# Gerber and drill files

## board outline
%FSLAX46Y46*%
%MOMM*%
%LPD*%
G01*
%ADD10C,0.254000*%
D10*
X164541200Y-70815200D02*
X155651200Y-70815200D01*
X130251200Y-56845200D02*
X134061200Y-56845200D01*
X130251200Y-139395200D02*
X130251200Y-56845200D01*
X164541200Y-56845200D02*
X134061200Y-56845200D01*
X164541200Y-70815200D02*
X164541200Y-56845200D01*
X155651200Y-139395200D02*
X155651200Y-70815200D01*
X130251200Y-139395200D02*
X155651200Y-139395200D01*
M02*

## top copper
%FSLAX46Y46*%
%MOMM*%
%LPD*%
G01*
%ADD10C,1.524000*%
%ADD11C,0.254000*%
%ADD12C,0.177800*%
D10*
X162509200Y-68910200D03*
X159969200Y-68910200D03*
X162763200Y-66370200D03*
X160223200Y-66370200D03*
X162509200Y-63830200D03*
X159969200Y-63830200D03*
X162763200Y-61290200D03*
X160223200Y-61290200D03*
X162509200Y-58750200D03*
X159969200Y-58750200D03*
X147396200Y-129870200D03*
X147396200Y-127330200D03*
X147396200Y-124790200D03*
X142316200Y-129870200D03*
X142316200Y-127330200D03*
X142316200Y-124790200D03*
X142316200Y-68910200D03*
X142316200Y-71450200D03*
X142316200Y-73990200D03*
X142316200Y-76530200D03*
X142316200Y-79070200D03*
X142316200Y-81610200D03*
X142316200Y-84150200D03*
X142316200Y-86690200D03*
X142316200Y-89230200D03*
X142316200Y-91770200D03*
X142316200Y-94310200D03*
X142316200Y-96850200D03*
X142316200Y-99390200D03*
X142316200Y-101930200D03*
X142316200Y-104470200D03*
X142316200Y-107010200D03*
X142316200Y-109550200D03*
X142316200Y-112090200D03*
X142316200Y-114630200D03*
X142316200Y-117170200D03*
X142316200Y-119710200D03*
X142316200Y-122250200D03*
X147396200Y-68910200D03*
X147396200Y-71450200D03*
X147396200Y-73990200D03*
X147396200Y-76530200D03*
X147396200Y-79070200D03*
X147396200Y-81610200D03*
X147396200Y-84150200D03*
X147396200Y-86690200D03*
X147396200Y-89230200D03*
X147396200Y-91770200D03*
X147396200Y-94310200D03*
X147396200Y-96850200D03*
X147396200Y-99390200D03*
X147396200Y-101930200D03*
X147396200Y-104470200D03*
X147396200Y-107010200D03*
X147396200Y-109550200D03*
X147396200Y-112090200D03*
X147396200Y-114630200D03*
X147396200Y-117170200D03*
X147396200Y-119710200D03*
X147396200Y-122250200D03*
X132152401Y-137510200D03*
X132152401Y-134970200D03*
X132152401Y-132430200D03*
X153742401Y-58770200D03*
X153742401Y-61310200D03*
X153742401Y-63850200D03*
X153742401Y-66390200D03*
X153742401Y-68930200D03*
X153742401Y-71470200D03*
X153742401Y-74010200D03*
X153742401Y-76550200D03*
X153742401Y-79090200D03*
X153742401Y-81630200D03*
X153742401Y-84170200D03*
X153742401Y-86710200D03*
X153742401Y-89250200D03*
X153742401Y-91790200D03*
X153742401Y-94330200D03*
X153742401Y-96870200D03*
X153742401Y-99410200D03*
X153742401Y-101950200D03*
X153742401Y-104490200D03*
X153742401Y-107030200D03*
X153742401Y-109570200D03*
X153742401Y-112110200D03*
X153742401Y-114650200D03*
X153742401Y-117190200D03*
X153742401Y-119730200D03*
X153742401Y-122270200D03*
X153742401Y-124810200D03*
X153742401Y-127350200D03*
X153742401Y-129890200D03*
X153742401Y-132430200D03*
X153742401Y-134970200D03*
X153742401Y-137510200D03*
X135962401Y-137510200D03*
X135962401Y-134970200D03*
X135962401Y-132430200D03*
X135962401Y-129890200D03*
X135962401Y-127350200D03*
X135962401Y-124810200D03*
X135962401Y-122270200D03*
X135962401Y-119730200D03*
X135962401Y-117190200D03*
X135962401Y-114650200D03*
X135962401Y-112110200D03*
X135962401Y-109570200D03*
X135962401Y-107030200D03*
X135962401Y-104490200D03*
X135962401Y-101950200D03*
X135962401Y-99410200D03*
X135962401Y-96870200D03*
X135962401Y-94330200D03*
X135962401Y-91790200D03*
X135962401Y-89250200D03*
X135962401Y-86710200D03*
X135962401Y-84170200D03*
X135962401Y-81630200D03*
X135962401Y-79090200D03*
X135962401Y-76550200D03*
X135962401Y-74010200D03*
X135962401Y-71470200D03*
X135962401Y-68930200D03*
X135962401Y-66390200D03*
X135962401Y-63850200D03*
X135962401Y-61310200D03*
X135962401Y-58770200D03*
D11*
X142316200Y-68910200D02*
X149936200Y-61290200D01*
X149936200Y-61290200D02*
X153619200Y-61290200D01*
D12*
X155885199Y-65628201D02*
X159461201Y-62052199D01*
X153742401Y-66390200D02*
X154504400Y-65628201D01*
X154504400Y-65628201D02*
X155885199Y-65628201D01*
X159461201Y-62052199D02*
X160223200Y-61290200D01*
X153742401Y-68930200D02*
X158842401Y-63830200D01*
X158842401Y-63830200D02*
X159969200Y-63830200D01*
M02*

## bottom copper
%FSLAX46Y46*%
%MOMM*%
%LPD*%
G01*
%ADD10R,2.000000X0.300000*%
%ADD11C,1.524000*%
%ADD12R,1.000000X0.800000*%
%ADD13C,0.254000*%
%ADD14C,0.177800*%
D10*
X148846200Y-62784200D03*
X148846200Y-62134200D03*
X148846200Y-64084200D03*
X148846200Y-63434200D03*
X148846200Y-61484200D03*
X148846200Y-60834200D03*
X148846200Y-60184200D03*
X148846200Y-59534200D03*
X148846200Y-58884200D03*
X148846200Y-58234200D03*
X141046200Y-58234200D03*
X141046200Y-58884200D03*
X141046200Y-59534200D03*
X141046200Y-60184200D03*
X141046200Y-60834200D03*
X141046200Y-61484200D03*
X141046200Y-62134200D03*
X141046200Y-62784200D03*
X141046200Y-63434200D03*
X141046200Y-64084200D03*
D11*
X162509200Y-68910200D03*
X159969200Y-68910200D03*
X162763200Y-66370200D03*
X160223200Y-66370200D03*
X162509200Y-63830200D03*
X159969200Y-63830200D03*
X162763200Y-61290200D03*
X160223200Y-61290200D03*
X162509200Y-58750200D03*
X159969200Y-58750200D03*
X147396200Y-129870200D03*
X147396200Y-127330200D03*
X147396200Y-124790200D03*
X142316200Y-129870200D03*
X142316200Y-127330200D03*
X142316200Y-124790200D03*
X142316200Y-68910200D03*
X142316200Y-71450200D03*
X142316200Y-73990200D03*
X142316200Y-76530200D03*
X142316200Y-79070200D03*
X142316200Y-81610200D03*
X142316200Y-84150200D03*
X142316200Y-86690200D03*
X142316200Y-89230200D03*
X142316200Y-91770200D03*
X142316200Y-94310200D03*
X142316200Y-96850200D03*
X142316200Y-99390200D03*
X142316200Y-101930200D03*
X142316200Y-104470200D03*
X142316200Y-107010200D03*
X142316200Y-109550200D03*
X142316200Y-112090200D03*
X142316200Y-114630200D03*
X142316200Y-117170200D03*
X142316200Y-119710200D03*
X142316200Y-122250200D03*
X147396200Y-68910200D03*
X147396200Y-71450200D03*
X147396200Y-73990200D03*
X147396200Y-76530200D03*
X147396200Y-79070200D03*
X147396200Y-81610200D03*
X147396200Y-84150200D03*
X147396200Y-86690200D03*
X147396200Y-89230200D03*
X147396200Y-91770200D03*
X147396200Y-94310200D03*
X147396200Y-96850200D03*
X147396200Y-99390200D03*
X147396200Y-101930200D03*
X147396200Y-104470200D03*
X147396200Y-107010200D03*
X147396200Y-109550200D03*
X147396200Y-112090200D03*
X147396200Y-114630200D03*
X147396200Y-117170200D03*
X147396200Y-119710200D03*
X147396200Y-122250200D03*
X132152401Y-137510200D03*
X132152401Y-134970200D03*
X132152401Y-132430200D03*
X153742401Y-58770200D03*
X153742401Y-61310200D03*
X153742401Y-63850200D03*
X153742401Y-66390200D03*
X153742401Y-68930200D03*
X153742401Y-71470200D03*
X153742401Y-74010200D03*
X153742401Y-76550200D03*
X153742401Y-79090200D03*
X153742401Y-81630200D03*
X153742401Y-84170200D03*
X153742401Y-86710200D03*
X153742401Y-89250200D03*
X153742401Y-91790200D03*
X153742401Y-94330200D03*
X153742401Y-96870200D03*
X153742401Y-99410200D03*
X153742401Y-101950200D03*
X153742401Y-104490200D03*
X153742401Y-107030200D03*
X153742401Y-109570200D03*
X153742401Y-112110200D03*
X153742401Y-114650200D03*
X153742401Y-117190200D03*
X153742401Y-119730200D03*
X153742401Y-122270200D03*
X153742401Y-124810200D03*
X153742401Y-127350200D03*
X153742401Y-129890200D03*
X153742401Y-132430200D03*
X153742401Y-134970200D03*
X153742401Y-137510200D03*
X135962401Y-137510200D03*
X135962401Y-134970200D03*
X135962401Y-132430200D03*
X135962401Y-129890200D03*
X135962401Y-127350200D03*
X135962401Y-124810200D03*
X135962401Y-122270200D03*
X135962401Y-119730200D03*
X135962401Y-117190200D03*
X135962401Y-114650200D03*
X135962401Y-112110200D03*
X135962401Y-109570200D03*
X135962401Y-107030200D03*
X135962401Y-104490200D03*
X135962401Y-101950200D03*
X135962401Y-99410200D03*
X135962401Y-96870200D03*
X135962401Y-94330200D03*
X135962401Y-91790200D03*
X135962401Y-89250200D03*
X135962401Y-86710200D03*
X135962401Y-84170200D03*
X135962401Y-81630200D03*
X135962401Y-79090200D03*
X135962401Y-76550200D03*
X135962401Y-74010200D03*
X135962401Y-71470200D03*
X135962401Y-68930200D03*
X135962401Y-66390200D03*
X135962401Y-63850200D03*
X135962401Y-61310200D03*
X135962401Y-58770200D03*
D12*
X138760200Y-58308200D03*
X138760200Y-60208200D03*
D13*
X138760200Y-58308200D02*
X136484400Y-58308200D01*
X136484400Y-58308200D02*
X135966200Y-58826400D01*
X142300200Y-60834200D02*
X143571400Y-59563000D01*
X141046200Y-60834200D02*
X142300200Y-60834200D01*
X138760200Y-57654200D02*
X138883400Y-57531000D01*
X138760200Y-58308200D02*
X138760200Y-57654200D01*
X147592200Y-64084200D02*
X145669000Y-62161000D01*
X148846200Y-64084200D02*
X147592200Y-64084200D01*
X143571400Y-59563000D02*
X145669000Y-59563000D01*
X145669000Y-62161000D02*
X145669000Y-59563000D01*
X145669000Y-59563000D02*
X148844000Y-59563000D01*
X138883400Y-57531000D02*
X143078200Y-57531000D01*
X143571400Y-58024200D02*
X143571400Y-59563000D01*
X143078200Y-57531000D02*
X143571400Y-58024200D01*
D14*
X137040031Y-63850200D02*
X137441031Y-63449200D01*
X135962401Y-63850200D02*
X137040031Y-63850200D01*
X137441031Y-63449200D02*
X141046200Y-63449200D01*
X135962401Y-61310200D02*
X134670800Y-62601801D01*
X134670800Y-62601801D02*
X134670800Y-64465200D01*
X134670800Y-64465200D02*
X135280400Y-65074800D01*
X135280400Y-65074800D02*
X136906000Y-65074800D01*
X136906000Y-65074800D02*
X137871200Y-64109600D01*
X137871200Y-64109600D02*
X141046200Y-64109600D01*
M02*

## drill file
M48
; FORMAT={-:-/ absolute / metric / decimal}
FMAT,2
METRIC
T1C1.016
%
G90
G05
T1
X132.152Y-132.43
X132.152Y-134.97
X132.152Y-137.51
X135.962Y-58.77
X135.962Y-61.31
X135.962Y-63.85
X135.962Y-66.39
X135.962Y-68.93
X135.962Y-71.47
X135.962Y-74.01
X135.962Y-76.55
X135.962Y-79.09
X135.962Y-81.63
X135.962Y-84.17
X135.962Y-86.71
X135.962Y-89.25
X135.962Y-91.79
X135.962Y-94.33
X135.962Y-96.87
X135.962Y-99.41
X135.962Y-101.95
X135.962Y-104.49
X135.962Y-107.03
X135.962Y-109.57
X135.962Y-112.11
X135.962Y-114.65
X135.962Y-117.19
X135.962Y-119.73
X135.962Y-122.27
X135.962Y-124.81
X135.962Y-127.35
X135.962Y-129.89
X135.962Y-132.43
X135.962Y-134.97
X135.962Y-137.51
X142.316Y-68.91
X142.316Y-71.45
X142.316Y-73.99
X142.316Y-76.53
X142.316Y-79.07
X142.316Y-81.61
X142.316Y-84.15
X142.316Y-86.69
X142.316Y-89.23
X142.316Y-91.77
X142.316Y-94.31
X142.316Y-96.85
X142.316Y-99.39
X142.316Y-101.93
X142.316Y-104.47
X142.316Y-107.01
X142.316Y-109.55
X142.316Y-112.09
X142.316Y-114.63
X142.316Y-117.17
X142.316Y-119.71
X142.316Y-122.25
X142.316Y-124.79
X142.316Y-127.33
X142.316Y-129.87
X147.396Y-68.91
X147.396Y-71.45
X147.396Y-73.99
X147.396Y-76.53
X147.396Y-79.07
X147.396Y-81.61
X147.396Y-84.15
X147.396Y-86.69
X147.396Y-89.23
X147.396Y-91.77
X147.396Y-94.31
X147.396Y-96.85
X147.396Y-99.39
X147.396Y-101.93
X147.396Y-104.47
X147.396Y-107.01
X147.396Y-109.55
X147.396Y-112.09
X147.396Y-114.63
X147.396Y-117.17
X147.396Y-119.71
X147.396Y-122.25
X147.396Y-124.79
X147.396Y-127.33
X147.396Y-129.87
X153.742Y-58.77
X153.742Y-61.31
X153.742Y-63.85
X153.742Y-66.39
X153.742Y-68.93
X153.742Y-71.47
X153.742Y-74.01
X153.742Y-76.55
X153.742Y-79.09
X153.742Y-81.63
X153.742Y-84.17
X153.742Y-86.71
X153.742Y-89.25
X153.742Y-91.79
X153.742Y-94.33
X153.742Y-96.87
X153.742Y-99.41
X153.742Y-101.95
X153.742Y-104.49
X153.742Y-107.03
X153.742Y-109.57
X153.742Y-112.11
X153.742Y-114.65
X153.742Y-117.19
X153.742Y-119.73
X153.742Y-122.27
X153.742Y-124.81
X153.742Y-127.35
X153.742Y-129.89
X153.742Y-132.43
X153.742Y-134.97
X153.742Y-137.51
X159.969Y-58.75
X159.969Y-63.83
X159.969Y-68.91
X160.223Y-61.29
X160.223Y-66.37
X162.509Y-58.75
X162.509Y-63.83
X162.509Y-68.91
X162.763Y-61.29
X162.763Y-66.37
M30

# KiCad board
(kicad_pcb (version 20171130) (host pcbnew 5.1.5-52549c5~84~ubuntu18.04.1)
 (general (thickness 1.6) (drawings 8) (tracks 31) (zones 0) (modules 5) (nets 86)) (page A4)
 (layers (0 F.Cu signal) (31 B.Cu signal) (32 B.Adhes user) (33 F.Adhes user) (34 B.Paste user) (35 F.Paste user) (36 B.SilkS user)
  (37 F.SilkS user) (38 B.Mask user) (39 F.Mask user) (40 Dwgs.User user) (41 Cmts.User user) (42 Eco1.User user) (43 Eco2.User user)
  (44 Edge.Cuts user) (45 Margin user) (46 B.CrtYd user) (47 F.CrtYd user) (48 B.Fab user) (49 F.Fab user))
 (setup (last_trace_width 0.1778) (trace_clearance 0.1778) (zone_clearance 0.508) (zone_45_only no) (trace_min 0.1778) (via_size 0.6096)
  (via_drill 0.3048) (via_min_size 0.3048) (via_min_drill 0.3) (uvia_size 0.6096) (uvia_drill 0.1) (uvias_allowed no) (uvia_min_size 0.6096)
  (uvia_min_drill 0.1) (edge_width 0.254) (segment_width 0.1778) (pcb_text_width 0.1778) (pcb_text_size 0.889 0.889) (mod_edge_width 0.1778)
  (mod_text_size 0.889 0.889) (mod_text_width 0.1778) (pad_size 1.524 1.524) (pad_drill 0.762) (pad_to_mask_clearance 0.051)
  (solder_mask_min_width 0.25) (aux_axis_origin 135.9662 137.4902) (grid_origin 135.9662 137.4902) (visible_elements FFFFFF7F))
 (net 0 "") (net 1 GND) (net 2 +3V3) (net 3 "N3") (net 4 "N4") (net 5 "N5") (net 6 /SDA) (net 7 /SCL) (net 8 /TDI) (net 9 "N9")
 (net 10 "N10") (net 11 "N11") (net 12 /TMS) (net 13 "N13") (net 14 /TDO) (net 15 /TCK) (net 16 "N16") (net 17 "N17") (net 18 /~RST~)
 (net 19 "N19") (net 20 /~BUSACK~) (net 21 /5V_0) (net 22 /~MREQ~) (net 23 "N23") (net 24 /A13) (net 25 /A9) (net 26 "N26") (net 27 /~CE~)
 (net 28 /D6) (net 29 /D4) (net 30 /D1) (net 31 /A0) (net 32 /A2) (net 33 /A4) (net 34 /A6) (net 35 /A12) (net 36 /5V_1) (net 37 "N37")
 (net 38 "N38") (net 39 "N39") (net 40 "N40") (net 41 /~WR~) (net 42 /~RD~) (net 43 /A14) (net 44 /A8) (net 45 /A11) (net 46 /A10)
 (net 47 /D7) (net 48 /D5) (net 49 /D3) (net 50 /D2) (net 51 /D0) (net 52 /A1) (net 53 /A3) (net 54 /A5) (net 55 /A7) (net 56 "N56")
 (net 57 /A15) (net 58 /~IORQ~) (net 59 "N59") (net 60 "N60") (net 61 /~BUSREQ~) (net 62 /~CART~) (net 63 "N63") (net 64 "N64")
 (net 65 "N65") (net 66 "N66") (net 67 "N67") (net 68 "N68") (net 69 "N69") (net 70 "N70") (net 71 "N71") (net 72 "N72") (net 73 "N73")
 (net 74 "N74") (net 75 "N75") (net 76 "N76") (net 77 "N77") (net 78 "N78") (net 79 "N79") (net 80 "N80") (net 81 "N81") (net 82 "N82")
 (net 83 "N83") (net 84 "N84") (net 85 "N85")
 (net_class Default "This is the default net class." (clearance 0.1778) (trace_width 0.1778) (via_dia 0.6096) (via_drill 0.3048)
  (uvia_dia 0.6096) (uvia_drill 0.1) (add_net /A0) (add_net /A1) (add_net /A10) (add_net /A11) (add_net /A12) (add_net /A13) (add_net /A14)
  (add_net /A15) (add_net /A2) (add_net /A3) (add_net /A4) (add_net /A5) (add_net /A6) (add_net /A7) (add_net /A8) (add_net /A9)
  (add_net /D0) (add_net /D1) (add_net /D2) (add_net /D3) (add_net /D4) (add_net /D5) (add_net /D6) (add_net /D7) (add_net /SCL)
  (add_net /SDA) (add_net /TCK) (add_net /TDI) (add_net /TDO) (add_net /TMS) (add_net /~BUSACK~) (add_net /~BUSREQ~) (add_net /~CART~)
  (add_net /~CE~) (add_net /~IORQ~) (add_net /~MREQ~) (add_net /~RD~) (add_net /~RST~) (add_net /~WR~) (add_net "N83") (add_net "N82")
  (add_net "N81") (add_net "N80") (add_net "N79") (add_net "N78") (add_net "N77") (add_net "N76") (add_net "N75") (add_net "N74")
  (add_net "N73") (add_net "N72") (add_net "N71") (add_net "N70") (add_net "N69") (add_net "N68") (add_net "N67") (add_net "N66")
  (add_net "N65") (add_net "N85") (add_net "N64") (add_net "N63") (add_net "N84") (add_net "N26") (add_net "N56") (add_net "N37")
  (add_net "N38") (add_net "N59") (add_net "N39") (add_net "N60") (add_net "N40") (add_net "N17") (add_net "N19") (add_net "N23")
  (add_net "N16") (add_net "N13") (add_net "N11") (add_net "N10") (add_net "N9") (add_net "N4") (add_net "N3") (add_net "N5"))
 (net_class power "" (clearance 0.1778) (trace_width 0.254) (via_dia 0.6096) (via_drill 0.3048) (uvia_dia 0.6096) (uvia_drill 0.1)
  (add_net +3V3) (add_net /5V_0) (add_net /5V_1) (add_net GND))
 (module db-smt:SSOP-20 (layer B.Cu) (at 141.0462 64.0842) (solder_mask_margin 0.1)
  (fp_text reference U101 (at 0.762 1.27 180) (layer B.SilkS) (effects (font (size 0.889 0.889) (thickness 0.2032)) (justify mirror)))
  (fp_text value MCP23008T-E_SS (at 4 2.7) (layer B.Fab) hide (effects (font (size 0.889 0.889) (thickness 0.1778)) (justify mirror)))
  (pad 18 smd rect (at 7.8 -1.3) (size 2 0.3) (layers B.Cu B.Paste B.Mask) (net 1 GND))
  (pad 17 smd rect (at 7.8 -1.95) (size 2 0.3) (layers B.Cu B.Paste B.Mask) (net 1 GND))
  (pad 20 smd rect (at 7.8 0) (size 2 0.3) (layers B.Cu B.Paste B.Mask) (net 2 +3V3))
  (pad 19 smd rect (at 7.8 -0.65) (size 2 0.3) (layers B.Cu B.Paste B.Mask) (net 1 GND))
  (pad 16 smd rect (at 7.8 -2.6) (size 2 0.3) (layers B.Cu B.Paste B.Mask) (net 1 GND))
  (pad 15 smd rect (at 7.8 -3.25) (size 2 0.3) (layers B.Cu B.Paste B.Mask) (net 1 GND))
  (pad 14 smd rect (at 7.8 -3.9) (size 2 0.3) (layers B.Cu B.Paste B.Mask) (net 1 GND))
  (pad 13 smd rect (at 7.8 -4.55) (size 2 0.3) (layers B.Cu B.Paste B.Mask) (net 2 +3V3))
  (pad 12 smd rect (at 7.8 -5.2) (size 2 0.3) (layers B.Cu B.Paste B.Mask) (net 1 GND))
  (pad 11 smd rect (at 7.8 -5.85) (size 2 0.3) (layers B.Cu B.Paste B.Mask) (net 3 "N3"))
  (pad 10 smd rect (at 0 -5.85) (size 2 0.3) (layers B.Cu B.Paste B.Mask) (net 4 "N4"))
  (pad 9 smd rect (at 0 -5.2) (size 2 0.3) (layers B.Cu B.Paste B.Mask) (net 1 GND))
  (pad 8 smd rect (at 0 -4.55) (size 2 0.3) (layers B.Cu B.Paste B.Mask) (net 1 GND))
  (pad 7 smd rect (at 0 -3.9) (size 2 0.3) (layers B.Cu B.Paste B.Mask) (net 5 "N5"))
  (pad 6 smd rect (at 0 -3.25) (size 2 0.3) (layers B.Cu B.Paste B.Mask) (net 2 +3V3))
  (pad 5 smd rect (at 0 -2.6) (size 2 0.3) (layers B.Cu B.Paste B.Mask) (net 1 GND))
  (pad 4 smd rect (at 0 -1.95) (size 2 0.3) (layers B.Cu B.Paste B.Mask) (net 1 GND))
  (pad 3 smd rect (at 0 -1.3) (size 2 0.3) (layers B.Cu B.Paste B.Mask) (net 1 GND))
  (pad 2 smd rect (at 0 -0.65) (size 2 0.3) (layers B.Cu B.Paste B.Mask) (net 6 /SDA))
  (pad 1 smd rect (at 0 0) (size 2 0.3) (layers B.Cu B.Paste B.Mask) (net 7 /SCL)))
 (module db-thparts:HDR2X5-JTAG (layer F.Cu) (at 160.0962 58.7502) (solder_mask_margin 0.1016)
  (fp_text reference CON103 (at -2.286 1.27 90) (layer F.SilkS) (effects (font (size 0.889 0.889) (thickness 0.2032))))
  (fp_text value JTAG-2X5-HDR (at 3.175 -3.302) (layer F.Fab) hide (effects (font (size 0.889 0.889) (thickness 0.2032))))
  (pad 10 thru_hole circle (at 2.413 10.16) (size 1.524 1.524) (drill 1.016) (layers *.Cu *.Mask) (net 1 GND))
  (pad 9 thru_hole circle (at -0.127 10.16) (size 1.524 1.524) (drill 1.016) (layers *.Cu *.Mask) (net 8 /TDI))
  (pad 8 thru_hole circle (at 2.667 7.62) (size 1.524 1.524) (drill 1.016) (layers *.Cu *.Mask) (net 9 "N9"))
  (pad 7 thru_hole circle (at 0.127 7.62) (size 1.524 1.524) (drill 1.016) (layers *.Cu *.Mask) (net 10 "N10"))
  (pad 6 thru_hole circle (at 2.413 5.08) (size 1.524 1.524) (drill 1.016) (layers *.Cu *.Mask) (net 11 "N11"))
  (pad 5 thru_hole circle (at -0.127 5.08) (size 1.524 1.524) (drill 1.016) (layers *.Cu *.Mask) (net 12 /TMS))
  (pad 4 thru_hole circle (at 2.667 2.54) (size 1.524 1.524) (drill 1.016) (layers *.Cu *.Mask) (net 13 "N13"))
  (pad 3 thru_hole circle (at 0.127 2.54) (size 1.524 1.524) (drill 1.016) (layers *.Cu *.Mask) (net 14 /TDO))
  (pad 2 thru_hole circle (at 2.413 0) (size 1.524 1.524) (drill 1.016) (layers *.Cu *.Mask) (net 1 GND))
  (pad 1 thru_hole circle (at -0.127 0) (size 1.524 1.524) (drill 1.016) (layers *.Cu *.Mask) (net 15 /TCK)))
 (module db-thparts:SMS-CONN (layer F.Cu) (at 142.3162 68.9102) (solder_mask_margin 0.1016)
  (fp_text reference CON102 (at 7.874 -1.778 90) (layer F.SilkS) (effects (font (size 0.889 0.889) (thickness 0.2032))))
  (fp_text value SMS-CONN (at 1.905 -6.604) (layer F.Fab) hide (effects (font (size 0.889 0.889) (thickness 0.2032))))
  (pad 50 thru_hole circle (at 5.08 60.96 180) (size 1.524 1.524) (drill 1.016) (layers *.Cu *.Mask) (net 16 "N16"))
  (pad 48 thru_hole circle (at 5.08 58.42 180) (size 1.524 1.524) (drill 1.016) (layers *.Cu *.Mask) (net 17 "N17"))
  (pad 46 thru_hole circle (at 5.08 55.88 180) (size 1.524 1.524) (drill 1.016) (layers *.Cu *.Mask) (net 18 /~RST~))
  (pad 49 thru_hole circle (at 0 60.96 180) (size 1.524 1.524) (drill 1.016) (layers *.Cu *.Mask) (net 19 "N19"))
  (pad 47 thru_hole circle (at 0 58.42 180) (size 1.524 1.524) (drill 1.016) (layers *.Cu *.Mask) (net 15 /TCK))
  (pad 45 thru_hole circle (at 0 55.88 180) (size 1.524 1.524) (drill 1.016) (layers *.Cu *.Mask) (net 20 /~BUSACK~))
  (pad 1 thru_hole circle (at 0 0 180) (size 1.524 1.524) (drill 1.016) (layers *.Cu *.Mask) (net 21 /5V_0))
  (pad 3 thru_hole circle (at 0 2.54 180) (size 1.524 1.524) (drill 1.016) (layers *.Cu *.Mask) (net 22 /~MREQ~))
  (pad 5 thru_hole circle (at 0 5.08 180) (size 1.524 1.524) (drill 1.016) (layers *.Cu *.Mask) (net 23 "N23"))
  (pad 7 thru_hole circle (at 0 7.62 180) (size 1.524 1.524) (drill 1.016) (layers *.Cu *.Mask) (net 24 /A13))
  (pad 9 thru_hole circle (at 0 10.16 180) (size 1.524 1.524) (drill 1.016) (layers *.Cu *.Mask) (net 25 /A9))
  (pad 11 thru_hole circle (at 0 12.7 180) (size 1.524 1.524) (drill 1.016) (layers *.Cu *.Mask) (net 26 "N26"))
  (pad 13 thru_hole circle (at 0 15.24 180) (size 1.524 1.524) (drill 1.016) (layers *.Cu *.Mask) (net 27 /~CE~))
  (pad 15 thru_hole circle (at 0 17.78 180) (size 1.524 1.524) (drill 1.016) (layers *.Cu *.Mask) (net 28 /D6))
  (pad 17 thru_hole circle (at 0 20.32 180) (size 1.524 1.524) (drill 1.016) (layers *.Cu *.Mask) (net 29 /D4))
  (pad 19 thru_hole circle (at 0 22.86 180) (size 1.524 1.524) (drill 1.016) (layers *.Cu *.Mask) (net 1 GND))
  (pad 21 thru_hole circle (at 0 25.4 180) (size 1.524 1.524) (drill 1.016) (layers *.Cu *.Mask) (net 1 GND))
  (pad 23 thru_hole circle (at 0 27.94 180) (size 1.524 1.524) (drill 1.016) (layers *.Cu *.Mask) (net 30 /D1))
  (pad 25 thru_hole circle (at 0 30.48 180) (size 1.524 1.524) (drill 1.016) (layers *.Cu *.Mask) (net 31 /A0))
  (pad 27 thru_hole circle (at 0 33.02 180) (size 1.524 1.524) (drill 1.016) (layers *.Cu *.Mask) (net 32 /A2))
  (pad 29 thru_hole circle (at 0 35.56 180) (size 1.524 1.524) (drill 1.016) (layers *.Cu *.Mask) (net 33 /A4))
  (pad 31 thru_hole circle (at 0 38.1 180) (size 1.524 1.524) (drill 1.016) (layers *.Cu *.Mask) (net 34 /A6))
  (pad 33 thru_hole circle (at 0 40.64 180) (size 1.524 1.524) (drill 1.016) (layers *.Cu *.Mask) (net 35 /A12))
  (pad 35 thru_hole circle (at 0 43.18 180) (size 1.524 1.524) (drill 1.016) (layers *.Cu *.Mask) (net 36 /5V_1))
  (pad 37 thru_hole circle (at 0 45.72 180) (size 1.524 1.524) (drill 1.016) (layers *.Cu *.Mask) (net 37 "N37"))
  (pad 39 thru_hole circle (at 0 48.26 180) (size 1.524 1.524) (drill 1.016) (layers *.Cu *.Mask) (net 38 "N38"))
  (pad 41 thru_hole circle (at 0 50.8 180) (size 1.524 1.524) (drill 1.016) (layers *.Cu *.Mask) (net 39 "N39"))
  (pad 43 thru_hole circle (at 0 53.34 180) (size 1.524 1.524) (drill 1.016) (layers *.Cu *.Mask) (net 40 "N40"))
  (pad 2 thru_hole circle (at 5.08 0 180) (size 1.524 1.524) (drill 1.016) (layers *.Cu *.Mask) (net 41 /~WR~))
  (pad 4 thru_hole circle (at 5.08 2.54 180) (size 1.524 1.524) (drill 1.016) (layers *.Cu *.Mask) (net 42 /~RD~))
  (pad 6 thru_hole circle (at 5.08 5.08 180) (size 1.524 1.524) (drill 1.016) (layers *.Cu *.Mask) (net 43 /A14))
  (pad 8 thru_hole circle (at 5.08 7.62 180) (size 1.524 1.524) (drill 1.016) (layers *.Cu *.Mask) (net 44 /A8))
  (pad 10 thru_hole circle (at 5.08 10.16 180) (size 1.524 1.524) (drill 1.016) (layers *.Cu *.Mask) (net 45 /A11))
  (pad 12 thru_hole circle (at 5.08 12.7 180) (size 1.524 1.524) (drill 1.016) (layers *.Cu *.Mask) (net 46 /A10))
  (pad 14 thru_hole circle (at 5.08 15.24 180) (size 1.524 1.524) (drill 1.016) (layers *.Cu *.Mask) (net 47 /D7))
  (pad 16 thru_hole circle (at 5.08 17.78 180) (size 1.524 1.524) (drill 1.016) (layers *.Cu *.Mask) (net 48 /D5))
  (pad 18 thru_hole circle (at 5.08 20.32 180) (size 1.524 1.524) (drill 1.016) (layers *.Cu *.Mask) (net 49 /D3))
  (pad 20 thru_hole circle (at 5.08 22.86 180) (size 1.524 1.524) (drill 1.016) (layers *.Cu *.Mask) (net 1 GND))
  (pad 22 thru_hole circle (at 5.08 25.4 180) (size 1.524 1.524) (drill 1.016) (layers *.Cu *.Mask) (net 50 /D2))
  (pad 24 thru_hole circle (at 5.08 27.94 180) (size 1.524 1.524) (drill 1.016) (layers *.Cu *.Mask) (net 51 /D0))
  (pad 26 thru_hole circle (at 5.08 30.48 180) (size 1.524 1.524) (drill 1.016) (layers *.Cu *.Mask) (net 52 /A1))
  (pad 28 thru_hole circle (at 5.08 33.02 180) (size 1.524 1.524) (drill 1.016) (layers *.Cu *.Mask) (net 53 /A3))
  (pad 30 thru_hole circle (at 5.08 35.56 180) (size 1.524 1.524) (drill 1.016) (layers *.Cu *.Mask) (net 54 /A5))
  (pad 32 thru_hole circle (at 5.08 38.1 180) (size 1.524 1.524) (drill 1.016) (layers *.Cu *.Mask) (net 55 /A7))
  (pad 34 thru_hole circle (at 5.08 40.64 180) (size 1.524 1.524) (drill 1.016) (layers *.Cu *.Mask) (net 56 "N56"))
  (pad 36 thru_hole circle (at 5.08 43.18 180) (size 1.524 1.524) (drill 1.016) (layers *.Cu *.Mask) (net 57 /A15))
  (pad 38 thru_hole circle (at 5.08 45.72 180) (size 1.524 1.524) (drill 1.016) (layers *.Cu *.Mask) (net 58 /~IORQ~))
  (pad 40 thru_hole circle (at 5.08 48.26 180) (size 1.524 1.524) (drill 1.016) (layers *.Cu *.Mask) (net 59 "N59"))
  (pad 42 thru_hole circle (at 5.08 50.8 180) (size 1.524 1.524) (drill 1.016) (layers *.Cu *.Mask) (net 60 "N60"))
  (pad 44 thru_hole circle (at 5.08 53.34 180) (size 1.524 1.524) (drill 1.016) (layers *.Cu *.Mask) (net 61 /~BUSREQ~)))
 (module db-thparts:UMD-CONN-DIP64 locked (layer F.Cu) (at 135.962401 58.7702) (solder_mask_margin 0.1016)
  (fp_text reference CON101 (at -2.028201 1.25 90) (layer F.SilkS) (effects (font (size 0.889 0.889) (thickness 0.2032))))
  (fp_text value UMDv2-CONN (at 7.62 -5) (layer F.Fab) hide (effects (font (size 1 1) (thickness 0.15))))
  (pad 67 thru_hole circle (at -3.81 78.74 270) (size 1.524 1.524) (drill 1.016) (layers *.Cu *.Mask) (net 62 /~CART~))
  (pad 66 thru_hole circle (at -3.81 76.2 270) (size 1.524 1.524) (drill 1.016) (layers *.Cu *.Mask) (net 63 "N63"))
  (pad 65 thru_hole circle (at -3.81 73.66 270) (size 1.524 1.524) (drill 1.016) (layers *.Cu *.Mask) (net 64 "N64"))
  (pad 64 thru_hole circle (at 17.78 0) (size 1.524 1.524) (drill 1.016) (layers *.Cu *.Mask) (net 1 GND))
  (pad 63 thru_hole circle (at 17.78 2.54) (size 1.524 1.524) (drill 1.016) (layers *.Cu *.Mask) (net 21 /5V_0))
  (pad 62 thru_hole circle (at 17.78 5.08) (size 1.524 1.524) (drill 1.016) (layers *.Cu *.Mask) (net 18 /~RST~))
  (pad 61 thru_hole circle (at 17.78 7.62) (size 1.524 1.524) (drill 1.016) (layers *.Cu *.Mask) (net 14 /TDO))
  (pad 60 thru_hole circle (at 17.78 10.16) (size 1.524 1.524) (drill 1.016) (layers *.Cu *.Mask) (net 12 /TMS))
  (pad 59 thru_hole circle (at 17.78 12.7) (size 1.524 1.524) (drill 1.016) (layers *.Cu *.Mask) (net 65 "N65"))
  (pad 58 thru_hole circle (at 17.78 15.24) (size 1.524 1.524) (drill 1.016) (layers *.Cu *.Mask) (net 43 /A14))
  (pad 57 thru_hole circle (at 17.78 17.78) (size 1.524 1.524) (drill 1.016) (layers *.Cu *.Mask) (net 35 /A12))
  (pad 56 thru_hole circle (at 17.78 20.32) (size 1.524 1.524) (drill 1.016) (layers *.Cu *.Mask) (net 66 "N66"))
  (pad 55 thru_hole circle (at 17.78 22.86) (size 1.524 1.524) (drill 1.016) (layers *.Cu *.Mask) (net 42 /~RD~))
  (pad 54 thru_hole circle (at 17.78 25.4) (size 1.524 1.524) (drill 1.016) (layers *.Cu *.Mask) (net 45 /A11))
  (pad 53 thru_hole circle (at 17.78 27.94) (size 1.524 1.524) (drill 1.016) (layers *.Cu *.Mask) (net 25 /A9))
  (pad 52 thru_hole circle (at 17.78 30.48) (size 1.524 1.524) (drill 1.016) (layers *.Cu *.Mask) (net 55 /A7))
  (pad 51 thru_hole circle (at 17.78 33.02) (size 1.524 1.524) (drill 1.016) (layers *.Cu *.Mask) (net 30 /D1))
  (pad 50 thru_hole circle (at 17.78 35.56) (size 1.524 1.524) (drill 1.016) (layers *.Cu *.Mask) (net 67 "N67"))
  (pad 49 thru_hole circle (at 17.78 38.1) (size 1.524 1.524) (drill 1.016) (layers *.Cu *.Mask) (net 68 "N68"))
  (pad 48 thru_hole circle (at 17.78 40.64) (size 1.524 1.524) (drill 1.016) (layers *.Cu *.Mask) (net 49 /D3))
  (pad 47 thru_hole circle (at 17.78 43.18) (size 1.524 1.524) (drill 1.016) (layers *.Cu *.Mask) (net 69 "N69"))
  (pad 46 thru_hole circle (at 17.78 45.72) (size 1.524 1.524) (drill 1.016) (layers *.Cu *.Mask) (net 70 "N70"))
  (pad 45 thru_hole circle (at 17.78 48.26) (size 1.524 1.524) (drill 1.016) (layers *.Cu *.Mask) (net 47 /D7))
  (pad 44 thru_hole circle (at 17.78 50.8) (size 1.524 1.524) (drill 1.016) (layers *.Cu *.Mask) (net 48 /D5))
  (pad 43 thru_hole circle (at 17.78 53.34) (size 1.524 1.524) (drill 1.016) (layers *.Cu *.Mask) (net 58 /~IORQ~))
  (pad 42 thru_hole circle (at 17.78 55.88) (size 1.524 1.524) (drill 1.016) (layers *.Cu *.Mask) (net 61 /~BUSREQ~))
  (pad 41 thru_hole circle (at 17.78 58.42) (size 1.524 1.524) (drill 1.016) (layers *.Cu *.Mask) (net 34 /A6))
  (pad 40 thru_hole circle (at 17.78 60.96) (size 1.524 1.524) (drill 1.016) (layers *.Cu *.Mask) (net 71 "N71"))
  (pad 39 thru_hole circle (at 17.78 63.5) (size 1.524 1.524) (drill 1.016) (layers *.Cu *.Mask) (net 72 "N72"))
  (pad 38 thru_hole circle (at 17.78 66.04) (size 1.524 1.524) (drill 1.016) (layers *.Cu *.Mask) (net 33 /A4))
  (pad 37 thru_hole circle (at 17.78 68.58) (size 1.524 1.524) (drill 1.016) (layers *.Cu *.Mask) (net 32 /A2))
  (pad 36 thru_hole circle (at 17.78 71.12) (size 1.524 1.524) (drill 1.016) (layers *.Cu *.Mask) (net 31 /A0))
  (pad 35 thru_hole circle (at 17.78 73.66) (size 1.524 1.524) (drill 1.016) (layers *.Cu *.Mask) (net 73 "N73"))
  (pad 34 thru_hole circle (at 17.78 76.2) (size 1.524 1.524) (drill 1.016) (layers *.Cu *.Mask) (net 36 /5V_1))
  (pad 33 thru_hole circle (at 17.78 78.74) (size 1.524 1.524) (drill 1.016) (layers *.Cu *.Mask) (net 1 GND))
  (pad 32 thru_hole circle (at 0 78.74) (size 1.524 1.524) (drill 1.016) (layers *.Cu *.Mask) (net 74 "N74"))
  (pad 31 thru_hole circle (at 0 76.2) (size 1.524 1.524) (drill 1.016) (layers *.Cu *.Mask) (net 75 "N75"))
  (pad 30 thru_hole circle (at 0 73.66) (size 1.524 1.524) (drill 1.016) (layers *.Cu *.Mask) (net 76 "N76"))
  (pad 29 thru_hole circle (at 0 71.12) (size 1.524 1.524) (drill 1.016) (layers *.Cu *.Mask) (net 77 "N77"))
  (pad 28 thru_hole circle (at 0 68.58) (size 1.524 1.524) (drill 1.016) (layers *.Cu *.Mask) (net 52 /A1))
  (pad 27 thru_hole circle (at 0 66.04) (size 1.524 1.524) (drill 1.016) (layers *.Cu *.Mask) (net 53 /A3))
  (pad 26 thru_hole circle (at 0 63.5) (size 1.524 1.524) (drill 1.016) (layers *.Cu *.Mask) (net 54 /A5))
  (pad 25 thru_hole circle (at 0 60.96) (size 1.524 1.524) (drill 1.016) (layers *.Cu *.Mask) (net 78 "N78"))
  (pad 24 thru_hole circle (at 0 58.42) (size 1.524 1.524) (drill 1.016) (layers *.Cu *.Mask) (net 27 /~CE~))
  (pad 23 thru_hole circle (at 0 55.88) (size 1.524 1.524) (drill 1.016) (layers *.Cu *.Mask) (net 20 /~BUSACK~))
  (pad 22 thru_hole circle (at 0 53.34) (size 1.524 1.524) (drill 1.016) (layers *.Cu *.Mask) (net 22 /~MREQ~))
  (pad 21 thru_hole circle (at 0 50.8) (size 1.524 1.524) (drill 1.016) (layers *.Cu *.Mask) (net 29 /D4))
  (pad 20 thru_hole circle (at 0 48.26) (size 1.524 1.524) (drill 1.016) (layers *.Cu *.Mask) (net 28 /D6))
  (pad 19 thru_hole circle (at 0 45.72) (size 1.524 1.524) (drill 1.016) (layers *.Cu *.Mask) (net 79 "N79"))
  (pad 18 thru_hole circle (at 0 43.18) (size 1.524 1.524) (drill 1.016) (layers *.Cu *.Mask) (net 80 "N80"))
  (pad 17 thru_hole circle (at 0 40.64) (size 1.524 1.524) (drill 1.016) (layers *.Cu *.Mask) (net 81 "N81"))
  (pad 16 thru_hole circle (at 0 38.1) (size 1.524 1.524) (drill 1.016) (layers *.Cu *.Mask) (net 50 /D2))
  (pad 15 thru_hole circle (at 0 35.56) (size 1.524 1.524) (drill 1.016) (layers *.Cu *.Mask) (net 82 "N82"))
  (pad 14 thru_hole circle (at 0 33.02) (size 1.524 1.524) (drill 1.016) (layers *.Cu *.Mask) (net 51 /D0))
  (pad 13 thru_hole circle (at 0 30.48) (size 1.524 1.524) (drill 1.016) (layers *.Cu *.Mask) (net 44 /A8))
  (pad 12 thru_hole circle (at 0 27.94) (size 1.524 1.524) (drill 1.016) (layers *.Cu *.Mask) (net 46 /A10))
  (pad 11 thru_hole circle (at 0 25.4) (size 1.524 1.524) (drill 1.016) (layers *.Cu *.Mask) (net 41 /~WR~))
  (pad 10 thru_hole circle (at 0 22.86) (size 1.524 1.524) (drill 1.016) (layers *.Cu *.Mask) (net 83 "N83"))
  (pad 9 thru_hole circle (at 0 20.32) (size 1.524 1.524) (drill 1.016) (layers *.Cu *.Mask) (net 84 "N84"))
  (pad 8 thru_hole circle (at 0 17.78) (size 1.524 1.524) (drill 1.016) (layers *.Cu *.Mask) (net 24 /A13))
  (pad 7 thru_hole circle (at 0 15.24) (size 1.524 1.524) (drill 1.016) (layers *.Cu *.Mask) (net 57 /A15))
  (pad 6 thru_hole circle (at 0 12.7) (size 1.524 1.524) (drill 1.016) (layers *.Cu *.Mask) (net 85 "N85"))
  (pad 5 thru_hole circle (at 0 10.16) (size 1.524 1.524) (drill 1.016) (layers *.Cu *.Mask) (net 15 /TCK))
  (pad 4 thru_hole circle (at 0 7.62) (size 1.524 1.524) (drill 1.016) (layers *.Cu *.Mask) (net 8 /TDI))
  (pad 3 thru_hole circle (at 0 5.08) (size 1.524 1.524) (drill 1.016) (layers *.Cu *.Mask) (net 6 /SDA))
  (pad 2 thru_hole circle (at 0 2.54) (size 1.524 1.524) (drill 1.016) (layers *.Cu *.Mask) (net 7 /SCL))
  (pad 1 thru_hole circle (at 0 0) (size 1.524 1.524) (drill 1.016) (layers *.Cu *.Mask) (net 2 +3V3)))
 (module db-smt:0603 (layer B.Cu) (at 138.7602 59.2582 270) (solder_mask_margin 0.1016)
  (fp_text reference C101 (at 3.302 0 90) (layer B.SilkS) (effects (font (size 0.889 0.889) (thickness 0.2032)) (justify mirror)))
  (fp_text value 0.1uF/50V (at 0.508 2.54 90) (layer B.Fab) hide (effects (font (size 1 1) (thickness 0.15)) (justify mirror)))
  (pad 1 smd rect (at -0.95 0 270) (size 0.8 1) (layers B.Cu B.Paste B.Mask) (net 2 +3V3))
  (pad 2 smd rect (at 0.95 0 270) (size 0.8 1) (layers B.Cu B.Paste B.Mask) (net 1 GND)))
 (gr_line (start 164.5412 70.8152) (end 155.6512 70.8152) (layer Edge.Cuts) (width 0.254))
 (gr_line (start 130.2512 56.8452) (end 134.0612 56.8452) (layer Edge.Cuts) (width 0.254))
 (gr_line (start 130.2512 139.3952) (end 130.2512 56.8452) (layer Edge.Cuts) (width 0.254))
 (gr_line (start 164.5412 56.8452) (end 134.0612 56.8452) (layer Edge.Cuts) (width 0.254))
 (gr_line (start 164.5412 70.8152) (end 164.5412 56.8452) (layer Edge.Cuts) (width 0.254))
 (gr_line (start 155.6512 139.3952) (end 155.6512 70.8152) (layer Edge.Cuts) (width 0.254))
 (gr_line (start 130.2512 139.3952) (end 155.6512 139.3952) (layer Edge.Cuts) (width 0.254))
 (segment (start 138.7602 58.3082) (end 136.4844 58.3082) (width 0.254) (layer B.Cu) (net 2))
 (segment (start 136.4844 58.3082) (end 135.9662 58.8264) (width 0.254) (layer B.Cu) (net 2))
 (segment (start 142.3002 60.8342) (end 143.5714 59.563) (width 0.254) (layer B.Cu) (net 2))
 (segment (start 141.0462 60.8342) (end 142.3002 60.8342) (width 0.254) (layer B.Cu) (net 2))
 (segment (start 138.7602 57.6542) (end 138.8834 57.531) (width 0.254) (layer B.Cu) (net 2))
 (segment (start 138.7602 58.3082) (end 138.7602 57.6542) (width 0.254) (layer B.Cu) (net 2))
 (segment (start 147.5922 64.0842) (end 145.669 62.161) (width 0.254) (layer B.Cu) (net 2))
 (segment (start 148.8462 64.0842) (end 147.5922 64.0842) (width 0.254) (layer B.Cu) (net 2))
 (segment (start 143.5714 59.563) (end 145.669 59.563) (width 0.254) (layer B.Cu) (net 2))
 (segment (start 145.669 62.161) (end 145.669 59.563) (width 0.254) (layer B.Cu) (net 2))
 (segment (start 145.669 59.563) (end 148.844 59.563) (width 0.254) (layer B.Cu) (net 2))
 (segment (start 138.8834 57.531) (end 143.0782 57.531) (width 0.254) (layer B.Cu) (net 2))
 (segment (start 143.5714 58.0242) (end 143.5714 59.563) (width 0.254) (layer B.Cu) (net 2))
 (segment (start 143.0782 57.531) (end 143.5714 58.0242) (width 0.254) (layer B.Cu) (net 2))
 (segment (start 142.3162 68.9102) (end 149.9362 61.2902) (width 0.254) (layer F.Cu) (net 21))
 (segment (start 149.9362 61.2902) (end 153.6192 61.2902) (width 0.254) (layer F.Cu) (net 21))
 (segment (start 155.885199 65.628201) (end 159.461201 62.052199) (width 0.1778) (layer F.Cu) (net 14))
 (segment (start 153.742401 66.3902) (end 154.5044 65.628201) (width 0.1778) (layer F.Cu) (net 14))
 (segment (start 154.5044 65.628201) (end 155.885199 65.628201) (width 0.1778) (layer F.Cu) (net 14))
 (segment (start 159.461201 62.052199) (end 160.2232 61.2902) (width 0.1778) (layer F.Cu) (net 14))
 (segment (start 153.742401 68.9302) (end 158.842401 63.8302) (width 0.1778) (layer F.Cu) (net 12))
 (segment (start 158.842401 63.8302) (end 159.9692 63.8302) (width 0.1778) (layer F.Cu) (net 12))
 (segment (start 137.040031 63.8502) (end 137.441031 63.4492) (width 0.1778) (layer B.Cu) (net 6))
 (segment (start 135.962401 63.8502) (end 137.040031 63.8502) (width 0.1778) (layer B.Cu) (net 6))
 (segment (start 137.441031 63.4492) (end 141.0462 63.4492) (width 0.1778) (layer B.Cu) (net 6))
 (segment (start 135.962401 61.3102) (end 134.6708 62.601801) (width 0.1778) (layer B.Cu) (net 7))
 (segment (start 134.6708 62.601801) (end 134.6708 64.4652) (width 0.1778) (layer B.Cu) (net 7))
 (segment (start 134.6708 64.4652) (end 135.2804 65.0748) (width 0.1778) (layer B.Cu) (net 7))
 (segment (start 135.2804 65.0748) (end 136.906 65.0748) (width 0.1778) (layer B.Cu) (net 7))
 (segment (start 136.906 65.0748) (end 137.8712 64.1096) (width 0.1778) (layer B.Cu) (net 7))
 (segment (start 137.8712 64.1096) (end 141.0462 64.1096) (width 0.1778) (layer B.Cu) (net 7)))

